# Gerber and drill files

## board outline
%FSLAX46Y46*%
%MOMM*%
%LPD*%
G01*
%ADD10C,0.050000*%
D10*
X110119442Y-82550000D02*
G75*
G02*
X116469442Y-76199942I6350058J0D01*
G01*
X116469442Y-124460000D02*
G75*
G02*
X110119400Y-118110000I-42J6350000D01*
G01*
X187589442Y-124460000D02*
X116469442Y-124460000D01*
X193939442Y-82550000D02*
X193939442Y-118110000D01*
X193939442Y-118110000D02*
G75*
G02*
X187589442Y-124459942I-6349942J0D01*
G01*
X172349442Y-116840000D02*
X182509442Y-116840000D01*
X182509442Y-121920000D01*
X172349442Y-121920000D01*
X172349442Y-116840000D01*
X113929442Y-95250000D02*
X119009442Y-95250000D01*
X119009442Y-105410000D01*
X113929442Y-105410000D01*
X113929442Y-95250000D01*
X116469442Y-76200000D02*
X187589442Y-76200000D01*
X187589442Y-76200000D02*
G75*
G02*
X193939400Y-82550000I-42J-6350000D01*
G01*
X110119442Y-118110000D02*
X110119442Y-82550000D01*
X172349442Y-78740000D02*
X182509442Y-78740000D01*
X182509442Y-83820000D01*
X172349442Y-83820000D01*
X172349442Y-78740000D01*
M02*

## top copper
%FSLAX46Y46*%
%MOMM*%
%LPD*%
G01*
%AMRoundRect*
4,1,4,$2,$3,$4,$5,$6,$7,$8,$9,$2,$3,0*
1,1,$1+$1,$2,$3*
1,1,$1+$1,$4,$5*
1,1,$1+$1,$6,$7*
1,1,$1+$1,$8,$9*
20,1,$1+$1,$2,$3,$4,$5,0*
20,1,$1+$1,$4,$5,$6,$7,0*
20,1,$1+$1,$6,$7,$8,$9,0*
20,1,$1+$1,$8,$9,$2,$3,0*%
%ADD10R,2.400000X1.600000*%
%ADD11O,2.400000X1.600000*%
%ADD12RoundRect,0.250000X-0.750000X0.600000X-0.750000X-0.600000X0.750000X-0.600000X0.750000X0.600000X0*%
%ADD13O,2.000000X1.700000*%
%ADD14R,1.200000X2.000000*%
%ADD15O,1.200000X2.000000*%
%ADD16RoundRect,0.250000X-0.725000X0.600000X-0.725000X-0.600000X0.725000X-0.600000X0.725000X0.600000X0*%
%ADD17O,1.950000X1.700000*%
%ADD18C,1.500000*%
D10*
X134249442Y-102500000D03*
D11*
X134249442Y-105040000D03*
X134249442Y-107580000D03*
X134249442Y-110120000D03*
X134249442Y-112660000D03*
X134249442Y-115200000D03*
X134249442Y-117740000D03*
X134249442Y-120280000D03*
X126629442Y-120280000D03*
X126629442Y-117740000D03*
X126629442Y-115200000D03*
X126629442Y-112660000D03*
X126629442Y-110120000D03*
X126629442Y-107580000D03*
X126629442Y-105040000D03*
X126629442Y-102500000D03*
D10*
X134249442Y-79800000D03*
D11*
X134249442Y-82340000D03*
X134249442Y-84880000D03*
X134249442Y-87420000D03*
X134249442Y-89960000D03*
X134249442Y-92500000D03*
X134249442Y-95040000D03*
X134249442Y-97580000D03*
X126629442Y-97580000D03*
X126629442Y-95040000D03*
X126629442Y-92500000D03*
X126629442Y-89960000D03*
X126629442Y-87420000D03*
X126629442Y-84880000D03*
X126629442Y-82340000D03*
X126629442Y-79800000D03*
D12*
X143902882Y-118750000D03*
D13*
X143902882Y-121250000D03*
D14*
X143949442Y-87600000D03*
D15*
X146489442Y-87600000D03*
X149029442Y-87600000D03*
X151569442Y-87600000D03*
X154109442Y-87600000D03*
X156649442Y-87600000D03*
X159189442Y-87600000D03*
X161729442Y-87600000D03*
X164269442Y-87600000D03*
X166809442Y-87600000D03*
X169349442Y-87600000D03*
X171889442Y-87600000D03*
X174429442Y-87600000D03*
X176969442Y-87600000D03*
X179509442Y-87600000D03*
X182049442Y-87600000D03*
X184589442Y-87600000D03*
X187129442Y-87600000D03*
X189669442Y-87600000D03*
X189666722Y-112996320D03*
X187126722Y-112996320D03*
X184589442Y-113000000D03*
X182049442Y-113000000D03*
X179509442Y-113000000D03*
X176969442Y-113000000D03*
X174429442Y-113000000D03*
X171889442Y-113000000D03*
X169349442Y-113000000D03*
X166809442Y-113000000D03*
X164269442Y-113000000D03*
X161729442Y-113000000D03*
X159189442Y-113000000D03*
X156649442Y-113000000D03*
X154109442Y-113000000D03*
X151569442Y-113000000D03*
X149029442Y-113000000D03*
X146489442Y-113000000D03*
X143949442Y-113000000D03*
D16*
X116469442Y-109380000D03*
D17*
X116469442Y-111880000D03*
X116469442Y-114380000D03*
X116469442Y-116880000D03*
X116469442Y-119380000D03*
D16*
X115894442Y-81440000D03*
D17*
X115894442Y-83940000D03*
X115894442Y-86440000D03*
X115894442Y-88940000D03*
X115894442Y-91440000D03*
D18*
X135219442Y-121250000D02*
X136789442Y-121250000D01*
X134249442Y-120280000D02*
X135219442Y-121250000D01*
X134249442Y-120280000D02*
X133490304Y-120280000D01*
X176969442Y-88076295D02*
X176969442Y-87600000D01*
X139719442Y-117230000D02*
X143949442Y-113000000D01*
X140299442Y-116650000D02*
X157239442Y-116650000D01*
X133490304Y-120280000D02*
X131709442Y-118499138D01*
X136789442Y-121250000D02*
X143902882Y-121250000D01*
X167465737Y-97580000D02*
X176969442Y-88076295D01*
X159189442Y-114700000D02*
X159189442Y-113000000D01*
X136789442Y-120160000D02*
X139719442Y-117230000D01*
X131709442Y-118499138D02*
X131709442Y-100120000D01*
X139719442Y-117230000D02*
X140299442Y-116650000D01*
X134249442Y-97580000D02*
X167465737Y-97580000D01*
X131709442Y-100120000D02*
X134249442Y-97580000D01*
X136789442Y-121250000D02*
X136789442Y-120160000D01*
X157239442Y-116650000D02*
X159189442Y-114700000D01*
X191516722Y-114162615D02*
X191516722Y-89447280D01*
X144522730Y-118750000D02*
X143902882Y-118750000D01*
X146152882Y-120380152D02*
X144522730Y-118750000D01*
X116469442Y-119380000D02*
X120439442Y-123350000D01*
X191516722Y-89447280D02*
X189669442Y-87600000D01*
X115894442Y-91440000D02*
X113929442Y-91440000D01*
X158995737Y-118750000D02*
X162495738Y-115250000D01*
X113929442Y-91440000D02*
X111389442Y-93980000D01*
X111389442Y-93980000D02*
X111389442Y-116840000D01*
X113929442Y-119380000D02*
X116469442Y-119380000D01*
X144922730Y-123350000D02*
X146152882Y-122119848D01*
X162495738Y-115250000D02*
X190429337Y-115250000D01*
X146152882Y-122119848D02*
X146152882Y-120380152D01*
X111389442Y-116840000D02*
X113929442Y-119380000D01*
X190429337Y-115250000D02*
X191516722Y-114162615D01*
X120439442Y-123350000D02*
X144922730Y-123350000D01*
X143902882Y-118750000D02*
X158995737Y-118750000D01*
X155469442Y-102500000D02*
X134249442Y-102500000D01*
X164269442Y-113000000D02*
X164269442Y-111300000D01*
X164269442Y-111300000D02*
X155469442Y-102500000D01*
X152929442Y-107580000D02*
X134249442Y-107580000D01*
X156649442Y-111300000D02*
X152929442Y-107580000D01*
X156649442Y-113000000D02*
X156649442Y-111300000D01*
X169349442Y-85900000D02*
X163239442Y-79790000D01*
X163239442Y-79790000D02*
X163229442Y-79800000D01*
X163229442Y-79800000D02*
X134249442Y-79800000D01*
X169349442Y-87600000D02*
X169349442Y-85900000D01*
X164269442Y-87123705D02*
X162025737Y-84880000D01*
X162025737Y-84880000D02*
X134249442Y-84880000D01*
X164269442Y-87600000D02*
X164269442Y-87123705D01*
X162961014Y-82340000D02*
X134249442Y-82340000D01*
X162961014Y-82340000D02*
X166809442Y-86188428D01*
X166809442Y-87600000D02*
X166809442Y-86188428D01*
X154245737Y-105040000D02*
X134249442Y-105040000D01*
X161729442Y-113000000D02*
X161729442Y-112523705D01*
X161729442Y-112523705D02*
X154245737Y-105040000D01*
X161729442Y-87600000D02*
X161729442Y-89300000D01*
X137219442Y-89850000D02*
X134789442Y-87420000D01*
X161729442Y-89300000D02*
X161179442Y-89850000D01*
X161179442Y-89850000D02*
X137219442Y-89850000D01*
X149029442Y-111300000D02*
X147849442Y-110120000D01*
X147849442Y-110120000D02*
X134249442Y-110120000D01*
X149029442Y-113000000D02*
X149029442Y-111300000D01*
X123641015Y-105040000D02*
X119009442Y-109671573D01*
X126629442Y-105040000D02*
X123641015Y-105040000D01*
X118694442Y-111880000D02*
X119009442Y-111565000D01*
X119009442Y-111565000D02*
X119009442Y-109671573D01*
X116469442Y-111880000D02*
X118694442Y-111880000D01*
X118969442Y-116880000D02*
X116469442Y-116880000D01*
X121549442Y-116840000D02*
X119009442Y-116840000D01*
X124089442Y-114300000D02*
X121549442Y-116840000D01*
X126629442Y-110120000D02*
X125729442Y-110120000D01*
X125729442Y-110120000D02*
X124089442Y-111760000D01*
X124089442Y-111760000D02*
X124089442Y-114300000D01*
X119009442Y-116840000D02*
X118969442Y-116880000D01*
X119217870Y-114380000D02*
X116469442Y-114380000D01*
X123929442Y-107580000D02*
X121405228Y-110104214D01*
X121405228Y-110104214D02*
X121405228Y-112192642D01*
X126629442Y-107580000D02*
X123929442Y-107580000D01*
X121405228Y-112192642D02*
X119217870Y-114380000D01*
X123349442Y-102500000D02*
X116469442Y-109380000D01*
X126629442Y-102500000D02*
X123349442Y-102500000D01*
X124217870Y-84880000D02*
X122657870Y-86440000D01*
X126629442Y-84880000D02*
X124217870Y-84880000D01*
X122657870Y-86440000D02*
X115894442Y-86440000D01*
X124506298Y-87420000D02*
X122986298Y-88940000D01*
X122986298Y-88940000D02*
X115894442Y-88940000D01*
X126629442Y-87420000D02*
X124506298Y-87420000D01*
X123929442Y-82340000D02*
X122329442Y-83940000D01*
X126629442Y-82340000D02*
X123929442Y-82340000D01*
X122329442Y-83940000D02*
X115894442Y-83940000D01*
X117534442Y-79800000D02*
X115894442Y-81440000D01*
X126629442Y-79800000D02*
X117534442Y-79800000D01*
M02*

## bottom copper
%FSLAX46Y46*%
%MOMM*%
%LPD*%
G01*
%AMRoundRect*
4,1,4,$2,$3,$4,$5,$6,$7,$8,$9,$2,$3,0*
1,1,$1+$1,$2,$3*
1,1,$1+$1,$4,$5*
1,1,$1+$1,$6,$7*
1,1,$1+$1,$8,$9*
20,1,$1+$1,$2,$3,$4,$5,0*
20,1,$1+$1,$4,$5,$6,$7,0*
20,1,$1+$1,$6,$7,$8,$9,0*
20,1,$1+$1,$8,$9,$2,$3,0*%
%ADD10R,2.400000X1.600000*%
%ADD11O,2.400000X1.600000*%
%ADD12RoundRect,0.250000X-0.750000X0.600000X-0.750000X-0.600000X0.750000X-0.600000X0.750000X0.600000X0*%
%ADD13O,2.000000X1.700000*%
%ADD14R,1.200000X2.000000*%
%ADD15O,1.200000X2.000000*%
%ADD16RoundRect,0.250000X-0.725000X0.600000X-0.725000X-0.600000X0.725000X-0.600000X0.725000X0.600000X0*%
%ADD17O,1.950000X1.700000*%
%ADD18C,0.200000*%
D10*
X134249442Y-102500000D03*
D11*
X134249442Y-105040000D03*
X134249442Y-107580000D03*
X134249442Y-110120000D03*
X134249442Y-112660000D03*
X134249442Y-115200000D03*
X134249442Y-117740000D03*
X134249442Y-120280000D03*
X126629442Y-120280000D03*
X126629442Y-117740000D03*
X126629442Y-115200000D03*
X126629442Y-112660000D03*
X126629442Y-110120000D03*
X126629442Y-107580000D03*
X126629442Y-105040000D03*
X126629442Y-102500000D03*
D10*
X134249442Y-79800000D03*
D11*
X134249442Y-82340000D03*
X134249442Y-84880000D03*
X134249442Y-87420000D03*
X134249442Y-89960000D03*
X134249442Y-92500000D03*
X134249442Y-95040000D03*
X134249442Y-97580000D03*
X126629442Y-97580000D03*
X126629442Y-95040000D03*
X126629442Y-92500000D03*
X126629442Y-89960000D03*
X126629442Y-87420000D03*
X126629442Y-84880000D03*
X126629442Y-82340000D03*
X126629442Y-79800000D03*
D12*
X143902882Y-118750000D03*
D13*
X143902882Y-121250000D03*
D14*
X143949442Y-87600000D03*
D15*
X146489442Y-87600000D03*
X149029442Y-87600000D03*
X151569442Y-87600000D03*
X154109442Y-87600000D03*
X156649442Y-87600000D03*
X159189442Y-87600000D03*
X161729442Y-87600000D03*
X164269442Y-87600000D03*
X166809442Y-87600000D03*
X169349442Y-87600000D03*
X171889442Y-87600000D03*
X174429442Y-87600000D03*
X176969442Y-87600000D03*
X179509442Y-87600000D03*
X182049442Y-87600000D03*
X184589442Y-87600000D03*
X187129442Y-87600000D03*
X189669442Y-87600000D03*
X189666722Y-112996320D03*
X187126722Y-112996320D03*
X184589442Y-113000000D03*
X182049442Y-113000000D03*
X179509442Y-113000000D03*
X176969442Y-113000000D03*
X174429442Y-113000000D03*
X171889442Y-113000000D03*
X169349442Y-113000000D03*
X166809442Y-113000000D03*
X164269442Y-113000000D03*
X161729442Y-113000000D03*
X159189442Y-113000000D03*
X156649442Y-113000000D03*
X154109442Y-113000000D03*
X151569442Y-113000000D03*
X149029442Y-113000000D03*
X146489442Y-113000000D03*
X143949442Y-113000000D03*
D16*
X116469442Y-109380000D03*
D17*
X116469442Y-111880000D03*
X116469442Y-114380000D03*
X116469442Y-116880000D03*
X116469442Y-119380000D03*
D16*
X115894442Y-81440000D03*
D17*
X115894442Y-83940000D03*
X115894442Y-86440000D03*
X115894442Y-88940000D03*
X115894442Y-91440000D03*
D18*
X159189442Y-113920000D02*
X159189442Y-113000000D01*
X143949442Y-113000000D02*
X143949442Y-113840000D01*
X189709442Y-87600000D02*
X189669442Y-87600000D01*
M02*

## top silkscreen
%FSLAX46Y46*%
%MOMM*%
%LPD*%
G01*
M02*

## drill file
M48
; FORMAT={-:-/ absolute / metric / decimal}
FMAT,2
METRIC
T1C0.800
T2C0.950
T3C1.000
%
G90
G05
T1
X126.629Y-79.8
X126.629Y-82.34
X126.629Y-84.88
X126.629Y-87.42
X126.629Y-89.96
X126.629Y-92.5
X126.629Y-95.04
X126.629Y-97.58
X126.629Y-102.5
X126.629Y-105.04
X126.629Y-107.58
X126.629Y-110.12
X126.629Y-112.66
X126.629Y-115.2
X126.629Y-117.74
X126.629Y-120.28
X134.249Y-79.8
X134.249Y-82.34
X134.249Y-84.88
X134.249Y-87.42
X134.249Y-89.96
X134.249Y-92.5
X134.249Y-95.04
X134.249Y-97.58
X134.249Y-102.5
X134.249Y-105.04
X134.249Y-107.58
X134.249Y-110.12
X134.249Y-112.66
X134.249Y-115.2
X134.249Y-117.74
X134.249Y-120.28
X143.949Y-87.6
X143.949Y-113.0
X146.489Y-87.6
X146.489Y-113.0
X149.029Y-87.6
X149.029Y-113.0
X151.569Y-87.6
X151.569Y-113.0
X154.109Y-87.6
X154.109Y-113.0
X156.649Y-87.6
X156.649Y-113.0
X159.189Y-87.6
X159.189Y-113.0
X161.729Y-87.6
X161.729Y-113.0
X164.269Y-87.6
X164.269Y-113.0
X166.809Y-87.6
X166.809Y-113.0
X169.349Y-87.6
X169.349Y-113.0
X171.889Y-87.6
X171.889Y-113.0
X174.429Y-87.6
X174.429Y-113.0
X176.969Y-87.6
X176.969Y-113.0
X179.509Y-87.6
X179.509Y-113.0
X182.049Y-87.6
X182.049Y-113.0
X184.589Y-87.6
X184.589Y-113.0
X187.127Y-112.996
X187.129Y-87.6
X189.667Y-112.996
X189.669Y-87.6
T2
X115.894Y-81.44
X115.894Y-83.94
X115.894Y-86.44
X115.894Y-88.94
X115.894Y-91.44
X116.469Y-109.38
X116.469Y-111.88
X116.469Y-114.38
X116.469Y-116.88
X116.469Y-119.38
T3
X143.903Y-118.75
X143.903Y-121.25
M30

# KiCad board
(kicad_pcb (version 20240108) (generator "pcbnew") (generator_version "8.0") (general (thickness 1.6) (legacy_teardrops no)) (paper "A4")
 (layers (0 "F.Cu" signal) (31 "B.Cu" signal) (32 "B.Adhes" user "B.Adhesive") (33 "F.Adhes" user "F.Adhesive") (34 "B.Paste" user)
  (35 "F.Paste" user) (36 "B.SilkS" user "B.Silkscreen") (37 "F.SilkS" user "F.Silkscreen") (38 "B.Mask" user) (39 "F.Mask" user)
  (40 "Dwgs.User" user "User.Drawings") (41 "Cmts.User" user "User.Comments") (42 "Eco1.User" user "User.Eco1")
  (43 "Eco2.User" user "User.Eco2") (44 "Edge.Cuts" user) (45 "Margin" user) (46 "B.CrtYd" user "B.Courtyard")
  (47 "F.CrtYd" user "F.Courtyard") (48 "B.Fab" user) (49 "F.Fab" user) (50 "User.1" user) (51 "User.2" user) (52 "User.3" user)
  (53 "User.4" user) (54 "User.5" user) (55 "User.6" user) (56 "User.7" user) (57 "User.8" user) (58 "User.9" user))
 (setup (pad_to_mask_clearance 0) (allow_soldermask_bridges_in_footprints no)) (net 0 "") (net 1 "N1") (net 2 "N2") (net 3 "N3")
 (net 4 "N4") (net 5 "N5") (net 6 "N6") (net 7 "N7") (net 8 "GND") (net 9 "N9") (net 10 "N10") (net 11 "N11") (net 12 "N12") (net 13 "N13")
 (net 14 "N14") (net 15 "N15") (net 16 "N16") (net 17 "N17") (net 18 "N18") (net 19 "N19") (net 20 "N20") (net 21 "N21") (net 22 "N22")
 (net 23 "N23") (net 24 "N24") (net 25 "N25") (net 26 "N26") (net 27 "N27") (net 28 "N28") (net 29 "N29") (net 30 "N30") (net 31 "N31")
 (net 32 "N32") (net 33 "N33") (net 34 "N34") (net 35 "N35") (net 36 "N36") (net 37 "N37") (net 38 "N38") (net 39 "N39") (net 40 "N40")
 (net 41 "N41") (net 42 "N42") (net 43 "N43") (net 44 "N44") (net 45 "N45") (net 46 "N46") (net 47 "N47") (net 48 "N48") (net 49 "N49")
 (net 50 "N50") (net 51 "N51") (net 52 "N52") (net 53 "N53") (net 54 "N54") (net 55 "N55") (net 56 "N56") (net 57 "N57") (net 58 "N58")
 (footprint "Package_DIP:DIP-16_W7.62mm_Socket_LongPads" (layer "B.Cu") (at 134.249442 102.5 180)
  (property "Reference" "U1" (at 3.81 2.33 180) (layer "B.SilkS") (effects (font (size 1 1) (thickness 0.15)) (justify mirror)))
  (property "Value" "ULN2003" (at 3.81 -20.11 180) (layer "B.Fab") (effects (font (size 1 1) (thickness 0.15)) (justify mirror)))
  (pad "1" thru_hole rect (at 0 0 180) (size 2.4 1.6) (drill 0.8) (layers "*.Cu" "*.Mask") (remove_unused_layers no) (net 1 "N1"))
  (pad "2" thru_hole oval (at 0 -2.54 180) (size 2.4 1.6) (drill 0.8) (layers "*.Cu" "*.Mask") (remove_unused_layers no) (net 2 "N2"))
  (pad "3" thru_hole oval (at 0 -5.08 180) (size 2.4 1.6) (drill 0.8) (layers "*.Cu" "*.Mask") (remove_unused_layers no) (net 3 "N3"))
  (pad "4" thru_hole oval (at 0 -7.62 180) (size 2.4 1.6) (drill 0.8) (layers "*.Cu" "*.Mask") (remove_unused_layers no) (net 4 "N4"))
  (pad "5" thru_hole oval (at 0 -10.16 180) (size 2.4 1.6) (drill 0.8) (layers "*.Cu" "*.Mask") (remove_unused_layers no) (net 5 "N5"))
  (pad "6" thru_hole oval (at 0 -12.7 180) (size 2.4 1.6) (drill 0.8) (layers "*.Cu" "*.Mask") (remove_unused_layers no) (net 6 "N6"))
  (pad "7" thru_hole oval (at 0 -15.24 180) (size 2.4 1.6) (drill 0.8) (layers "*.Cu" "*.Mask") (remove_unused_layers no) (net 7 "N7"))
  (pad "8" thru_hole oval (at 0 -17.78 180) (size 2.4 1.6) (drill 0.8) (layers "*.Cu" "*.Mask") (remove_unused_layers no) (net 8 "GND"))
  (pad "9" thru_hole oval (at 7.62 -17.78 180) (size 2.4 1.6) (drill 0.8) (layers "*.Cu" "*.Mask") (remove_unused_layers no) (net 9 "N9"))
  (pad "10" thru_hole oval (at 7.62 -15.24 180) (size 2.4 1.6) (drill 0.8) (layers "*.Cu" "*.Mask") (remove_unused_layers no) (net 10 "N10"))
  (pad "11" thru_hole oval (at 7.62 -12.7 180) (size 2.4 1.6) (drill 0.8) (layers "*.Cu" "*.Mask") (remove_unused_layers no) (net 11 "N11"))
  (pad "12" thru_hole oval (at 7.62 -10.16 180) (size 2.4 1.6) (drill 0.8) (layers "*.Cu" "*.Mask") (remove_unused_layers no) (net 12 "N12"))
  (pad "13" thru_hole oval (at 7.62 -7.62 180) (size 2.4 1.6) (drill 0.8) (layers "*.Cu" "*.Mask") (remove_unused_layers no) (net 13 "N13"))
  (pad "14" thru_hole oval (at 7.62 -5.08 180) (size 2.4 1.6) (drill 0.8) (layers "*.Cu" "*.Mask") (remove_unused_layers no) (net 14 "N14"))
  (pad "15" thru_hole oval (at 7.62 -2.54 180) (size 2.4 1.6) (drill 0.8) (layers "*.Cu" "*.Mask") (remove_unused_layers no) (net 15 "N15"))
  (pad "16" thru_hole oval (at 7.62 0 180) (size 2.4 1.6) (drill 0.8) (layers "*.Cu" "*.Mask") (remove_unused_layers no) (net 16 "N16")))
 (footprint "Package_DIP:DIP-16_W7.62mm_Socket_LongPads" (layer "B.Cu") (at 134.249442 79.8 180)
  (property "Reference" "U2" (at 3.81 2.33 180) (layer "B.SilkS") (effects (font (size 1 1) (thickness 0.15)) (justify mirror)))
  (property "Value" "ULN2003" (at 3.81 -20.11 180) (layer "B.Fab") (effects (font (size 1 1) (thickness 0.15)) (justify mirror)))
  (pad "1" thru_hole rect (at 0 0 180) (size 2.4 1.6) (drill 0.8) (layers "*.Cu" "*.Mask") (remove_unused_layers no) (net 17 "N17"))
  (pad "2" thru_hole oval (at 0 -2.54 180) (size 2.4 1.6) (drill 0.8) (layers "*.Cu" "*.Mask") (remove_unused_layers no) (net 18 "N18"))
  (pad "3" thru_hole oval (at 0 -5.08 180) (size 2.4 1.6) (drill 0.8) (layers "*.Cu" "*.Mask") (remove_unused_layers no) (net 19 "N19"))
  (pad "4" thru_hole oval (at 0 -7.62 180) (size 2.4 1.6) (drill 0.8) (layers "*.Cu" "*.Mask") (remove_unused_layers no) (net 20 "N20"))
  (pad "5" thru_hole oval (at 0 -10.16 180) (size 2.4 1.6) (drill 0.8) (layers "*.Cu" "*.Mask") (remove_unused_layers no) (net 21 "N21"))
  (pad "6" thru_hole oval (at 0 -12.7 180) (size 2.4 1.6) (drill 0.8) (layers "*.Cu" "*.Mask") (remove_unused_layers no) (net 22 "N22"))
  (pad "7" thru_hole oval (at 0 -15.24 180) (size 2.4 1.6) (drill 0.8) (layers "*.Cu" "*.Mask") (remove_unused_layers no) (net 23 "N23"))
  (pad "8" thru_hole oval (at 0 -17.78 180) (size 2.4 1.6) (drill 0.8) (layers "*.Cu" "*.Mask") (remove_unused_layers no) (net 8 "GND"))
  (pad "9" thru_hole oval (at 7.62 -17.78 180) (size 2.4 1.6) (drill 0.8) (layers "*.Cu" "*.Mask") (remove_unused_layers no) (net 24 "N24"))
  (pad "10" thru_hole oval (at 7.62 -15.24 180) (size 2.4 1.6) (drill 0.8) (layers "*.Cu" "*.Mask") (remove_unused_layers no) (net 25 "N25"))
  (pad "11" thru_hole oval (at 7.62 -12.7 180) (size 2.4 1.6) (drill 0.8) (layers "*.Cu" "*.Mask") (remove_unused_layers no) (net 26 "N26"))
  (pad "12" thru_hole oval (at 7.62 -10.16 180) (size 2.4 1.6) (drill 0.8) (layers "*.Cu" "*.Mask") (remove_unused_layers no) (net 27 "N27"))
  (pad "13" thru_hole oval (at 7.62 -7.62 180) (size 2.4 1.6) (drill 0.8) (layers "*.Cu" "*.Mask") (remove_unused_layers no) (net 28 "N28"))
  (pad "14" thru_hole oval (at 7.62 -5.08 180) (size 2.4 1.6) (drill 0.8) (layers "*.Cu" "*.Mask") (remove_unused_layers no) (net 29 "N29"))
  (pad "15" thru_hole oval (at 7.62 -2.54 180) (size 2.4 1.6) (drill 0.8) (layers "*.Cu" "*.Mask") (remove_unused_layers no) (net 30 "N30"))
  (pad "16" thru_hole oval (at 7.62 0 180) (size 2.4 1.6) (drill 0.8) (layers "*.Cu" "*.Mask") (remove_unused_layers no) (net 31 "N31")))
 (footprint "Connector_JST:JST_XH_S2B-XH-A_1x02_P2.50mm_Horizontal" (layer "B.Cu") (at 143.902882 118.75 -90)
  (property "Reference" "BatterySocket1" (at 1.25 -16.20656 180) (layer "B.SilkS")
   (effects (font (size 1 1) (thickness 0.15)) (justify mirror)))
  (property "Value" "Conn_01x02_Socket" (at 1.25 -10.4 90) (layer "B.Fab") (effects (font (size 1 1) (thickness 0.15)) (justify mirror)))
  (pad "1" thru_hole roundrect (at 0 0 270) (size 1.7 2) (drill 1) (layers "*.Cu" "*.Mask") (remove_unused_layers no)
   (roundrect_rratio 0.1470588235) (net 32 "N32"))
  (pad "2" thru_hole oval (at 2.5 0 270) (size 1.7 2) (drill 1) (layers "*.Cu" "*.Mask") (remove_unused_layers no) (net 8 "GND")))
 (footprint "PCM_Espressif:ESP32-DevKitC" (layer "B.Cu") (at 143.949442 87.6 -90)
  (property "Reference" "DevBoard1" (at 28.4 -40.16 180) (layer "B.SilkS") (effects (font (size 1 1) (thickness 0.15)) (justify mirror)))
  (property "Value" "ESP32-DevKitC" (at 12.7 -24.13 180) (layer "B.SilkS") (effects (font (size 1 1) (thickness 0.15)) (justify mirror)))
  (pad "1" thru_hole rect (at 0 0) (size 1.2 2) (drill 0.8) (layers "*.Cu" "*.Mask") (remove_unused_layers no) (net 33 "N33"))
  (pad "2" thru_hole oval (at 0 -2.54) (size 1.2 2) (drill 0.8) (layers "*.Cu" "*.Mask") (remove_unused_layers no) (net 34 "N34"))
  (pad "3" thru_hole oval (at 0 -5.08) (size 1.2 2) (drill 0.8) (layers "*.Cu" "*.Mask") (remove_unused_layers no) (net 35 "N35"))
  (pad "4" thru_hole oval (at 0 -7.62) (size 1.2 2) (drill 0.8) (layers "*.Cu" "*.Mask") (remove_unused_layers no) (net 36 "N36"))
  (pad "5" thru_hole oval (at 0 -10.16) (size 1.2 2) (drill 0.8) (layers "*.Cu" "*.Mask") (remove_unused_layers no) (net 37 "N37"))
  (pad "6" thru_hole oval (at 0 -12.7) (size 1.2 2) (drill 0.8) (layers "*.Cu" "*.Mask") (remove_unused_layers no) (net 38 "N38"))
  (pad "7" thru_hole oval (at 0 -15.24) (size 1.2 2) (drill 0.8) (layers "*.Cu" "*.Mask") (remove_unused_layers no) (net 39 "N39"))
  (pad "8" thru_hole oval (at 0 -17.78) (size 1.2 2) (drill 0.8) (layers "*.Cu" "*.Mask") (remove_unused_layers no) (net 20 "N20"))
  (pad "9" thru_hole oval (at 0 -20.32) (size 1.2 2) (drill 0.8) (layers "*.Cu" "*.Mask") (remove_unused_layers no) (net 19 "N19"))
  (pad "10" thru_hole oval (at 0 -22.86) (size 1.2 2) (drill 0.8) (layers "*.Cu" "*.Mask") (remove_unused_layers no) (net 18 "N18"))
  (pad "11" thru_hole oval (at 0 -25.4) (size 1.2 2) (drill 0.8) (layers "*.Cu" "*.Mask") (remove_unused_layers no) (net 17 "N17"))
  (pad "12" thru_hole oval (at 0 -27.94) (size 1.2 2) (drill 0.8) (layers "*.Cu" "*.Mask") (remove_unused_layers no) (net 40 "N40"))
  (pad "13" thru_hole oval (at 0 -30.48) (size 1.2 2) (drill 0.8) (layers "*.Cu" "*.Mask") (remove_unused_layers no) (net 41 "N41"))
  (pad "14" thru_hole oval (at 0 -33.02) (size 1.2 2) (drill 0.8) (layers "*.Cu" "*.Mask") (remove_unused_layers no) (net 8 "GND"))
  (pad "15" thru_hole oval (at 0 -35.56) (size 1.2 2) (drill 0.8) (layers "*.Cu" "*.Mask") (remove_unused_layers no) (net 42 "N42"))
  (pad "16" thru_hole oval (at 0 -38.1) (size 1.2 2) (drill 0.8) (layers "*.Cu" "*.Mask") (remove_unused_layers no) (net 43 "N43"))
  (pad "17" thru_hole oval (at 0 -40.64) (size 1.2 2) (drill 0.8) (layers "*.Cu" "*.Mask") (remove_unused_layers no) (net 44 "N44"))
  (pad "18" thru_hole oval (at 0 -43.18) (size 1.2 2) (drill 0.8) (layers "*.Cu" "*.Mask") (remove_unused_layers no) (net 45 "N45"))
  (pad "19" thru_hole oval (at 0 -45.72) (size 1.2 2) (drill 0.8) (layers "*.Cu" "*.Mask") (remove_unused_layers no) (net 32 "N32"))
  (pad "20" thru_hole oval (at 25.39632 -45.71728) (size 1.2 2) (drill 0.8) (layers "*.Cu" "*.Mask") (remove_unused_layers no)
   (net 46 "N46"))
  (pad "21" thru_hole oval (at 25.39632 -43.17728) (size 1.2 2) (drill 0.8) (layers "*.Cu" "*.Mask") (remove_unused_layers no)
   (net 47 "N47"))
  (pad "22" thru_hole oval (at 25.4 -40.64) (size 1.2 2) (drill 0.8) (layers "*.Cu" "*.Mask") (remove_unused_layers no) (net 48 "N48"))
  (pad "23" thru_hole oval (at 25.4 -38.1) (size 1.2 2) (drill 0.8) (layers "*.Cu" "*.Mask") (remove_unused_layers no) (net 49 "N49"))
  (pad "24" thru_hole oval (at 25.4 -35.56) (size 1.2 2) (drill 0.8) (layers "*.Cu" "*.Mask") (remove_unused_layers no) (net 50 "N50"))
  (pad "25" thru_hole oval (at 25.4 -33.02) (size 1.2 2) (drill 0.8) (layers "*.Cu" "*.Mask") (remove_unused_layers no) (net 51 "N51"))
  (pad "26" thru_hole oval (at 25.4 -30.48) (size 1.2 2) (drill 0.8) (layers "*.Cu" "*.Mask") (remove_unused_layers no) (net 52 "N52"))
  (pad "27" thru_hole oval (at 25.4 -27.94) (size 1.2 2) (drill 0.8) (layers "*.Cu" "*.Mask") (remove_unused_layers no) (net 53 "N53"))
  (pad "28" thru_hole oval (at 25.4 -25.4) (size 1.2 2) (drill 0.8) (layers "*.Cu" "*.Mask") (remove_unused_layers no) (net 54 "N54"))
  (pad "29" thru_hole oval (at 25.4 -22.86) (size 1.2 2) (drill 0.8) (layers "*.Cu" "*.Mask") (remove_unused_layers no) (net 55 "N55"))
  (pad "30" thru_hole oval (at 25.4 -20.32) (size 1.2 2) (drill 0.8) (layers "*.Cu" "*.Mask") (remove_unused_layers no) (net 1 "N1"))
  (pad "31" thru_hole oval (at 25.4 -17.78) (size 1.2 2) (drill 0.8) (layers "*.Cu" "*.Mask") (remove_unused_layers no) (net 2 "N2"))
  (pad "32" thru_hole oval (at 25.4 -15.24) (size 1.2 2) (drill 0.8) (layers "*.Cu" "*.Mask") (remove_unused_layers no) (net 8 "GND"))
  (pad "33" thru_hole oval (at 25.4 -12.7) (size 1.2 2) (drill 0.8) (layers "*.Cu" "*.Mask") (remove_unused_layers no) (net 3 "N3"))
  (pad "34" thru_hole oval (at 25.4 -10.16) (size 1.2 2) (drill 0.8) (layers "*.Cu" "*.Mask") (remove_unused_layers no) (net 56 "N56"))
  (pad "35" thru_hole oval (at 25.4 -7.62) (size 1.2 2) (drill 0.8) (layers "*.Cu" "*.Mask") (remove_unused_layers no) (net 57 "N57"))
  (pad "36" thru_hole oval (at 25.4 -5.08) (size 1.2 2) (drill 0.8) (layers "*.Cu" "*.Mask") (remove_unused_layers no) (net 4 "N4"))
  (pad "37" thru_hole oval (at 25.4 -2.54) (size 1.2 2) (drill 0.8) (layers "*.Cu" "*.Mask") (remove_unused_layers no) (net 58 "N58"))
  (pad "38" thru_hole oval (at 25.4 0) (size 1.2 2) (drill 0.8) (layers "*.Cu" "*.Mask") (remove_unused_layers no) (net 8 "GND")))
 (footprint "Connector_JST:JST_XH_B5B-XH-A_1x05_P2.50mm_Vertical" (layer "B.Cu") (at 116.469442 109.38 -90)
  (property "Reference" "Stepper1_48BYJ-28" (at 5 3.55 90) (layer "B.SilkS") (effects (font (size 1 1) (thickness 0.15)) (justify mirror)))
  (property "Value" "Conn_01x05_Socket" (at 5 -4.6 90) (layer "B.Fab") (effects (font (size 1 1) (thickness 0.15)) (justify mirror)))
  (pad "1" thru_hole roundrect (at 0 0 270) (size 1.7 1.95) (drill 0.95) (layers "*.Cu" "*.Mask") (remove_unused_layers no)
   (roundrect_rratio 0.1470588235) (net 16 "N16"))
  (pad "2" thru_hole oval (at 2.5 0 270) (size 1.7 1.95) (drill 0.95) (layers "*.Cu" "*.Mask") (remove_unused_layers no) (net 15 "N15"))
  (pad "3" thru_hole oval (at 5 0 270) (size 1.7 1.95) (drill 0.95) (layers "*.Cu" "*.Mask") (remove_unused_layers no) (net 14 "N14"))
  (pad "4" thru_hole oval (at 7.5 0 270) (size 1.7 1.95) (drill 0.95) (layers "*.Cu" "*.Mask") (remove_unused_layers no) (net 13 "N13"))
  (pad "5" thru_hole oval (at 10 0 270) (size 1.7 1.95) (drill 0.95) (layers "*.Cu" "*.Mask") (remove_unused_layers no) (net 32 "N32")))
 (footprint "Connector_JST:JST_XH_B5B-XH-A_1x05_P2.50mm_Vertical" (layer "B.Cu") (at 115.894442 81.44 -90)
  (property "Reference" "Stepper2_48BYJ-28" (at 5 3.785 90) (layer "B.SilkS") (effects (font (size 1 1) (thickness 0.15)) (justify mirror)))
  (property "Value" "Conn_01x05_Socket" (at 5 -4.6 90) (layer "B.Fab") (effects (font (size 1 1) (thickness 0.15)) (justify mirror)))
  (pad "1" thru_hole roundrect (at 0 0 270) (size 1.7 1.95) (drill 0.95) (layers "*.Cu" "*.Mask") (remove_unused_layers no)
   (roundrect_rratio 0.1470588235) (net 31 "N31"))
  (pad "2" thru_hole oval (at 2.5 0 270) (size 1.7 1.95) (drill 0.95) (layers "*.Cu" "*.Mask") (remove_unused_layers no) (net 30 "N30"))
  (pad "3" thru_hole oval (at 5 0 270) (size 1.7 1.95) (drill 0.95) (layers "*.Cu" "*.Mask") (remove_unused_layers no) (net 29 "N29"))
  (pad "4" thru_hole oval (at 7.5 0 270) (size 1.7 1.95) (drill 0.95) (layers "*.Cu" "*.Mask") (remove_unused_layers no) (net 28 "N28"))
  (pad "5" thru_hole oval (at 10 0 270) (size 1.7 1.95) (drill 0.95) (layers "*.Cu" "*.Mask") (remove_unused_layers no) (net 32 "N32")))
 (gr_arc (start 110.119442 82.55) (mid 111.979315 78.059877) (end 116.469442 76.2) (stroke (width 0.05) (type default)) (layer "Edge.Cuts"))
 (gr_arc (start 116.469442 124.46) (mid 111.979305 122.600133) (end 110.119442 118.11) (stroke (width 0.05) (type default))
  (layer "Edge.Cuts"))
 (gr_line (start 187.589442 124.46) (end 116.469442 124.46) (stroke (width 0.05) (type default)) (layer "Edge.Cuts"))
 (gr_line (start 193.939442 82.55) (end 193.939442 118.11) (stroke (width 0.05) (type default)) (layer "Edge.Cuts"))
 (gr_arc (start 193.939442 118.11) (mid 192.079571 122.600133) (end 187.589442 124.46) (stroke (width 0.05) (type default))
  (layer "Edge.Cuts"))
 (gr_rect (start 172.349442 116.84) (end 182.509442 121.92) (stroke (width 0.05) (type default)) (fill none) (layer "Edge.Cuts"))
 (gr_rect (start 113.929442 95.25) (end 119.009442 105.41) (stroke (width 0.05) (type default)) (fill none) (layer "Edge.Cuts"))
 (gr_line (start 116.469442 76.2) (end 187.589442 76.2) (stroke (width 0.05) (type default)) (layer "Edge.Cuts"))
 (gr_arc (start 187.589442 76.2) (mid 192.079561 78.059877) (end 193.939442 82.55) (stroke (width 0.05) (type default)) (layer "Edge.Cuts"))
 (gr_line (start 110.119442 118.11) (end 110.119442 82.55) (stroke (width 0.05) (type default)) (layer "Edge.Cuts"))
 (gr_rect (start 172.349442 78.74) (end 182.509442 83.82) (stroke (width 0.05) (type default)) (fill none) (layer "Edge.Cuts"))
 (segment (start 135.219442 121.25) (end 136.789442 121.25) (width 1.5) (layer "F.Cu") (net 8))
 (segment (start 134.249442 120.28) (end 135.219442 121.25) (width 1.5) (layer "F.Cu") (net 8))
 (segment (start 134.249442 120.28) (end 133.490304 120.28) (width 1.5) (layer "F.Cu") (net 8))
 (segment (start 176.969442 88.076295) (end 176.969442 87.6) (width 1.5) (layer "F.Cu") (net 8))
 (segment (start 139.719442 117.23) (end 143.949442 113) (width 1.5) (layer "F.Cu") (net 8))
 (segment (start 140.299442 116.65) (end 157.239442 116.65) (width 1.5) (layer "F.Cu") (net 8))
 (segment (start 133.490304 120.28) (end 131.709442 118.499138) (width 1.5) (layer "F.Cu") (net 8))
 (segment (start 136.789442 121.25) (end 143.902882 121.25) (width 1.5) (layer "F.Cu") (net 8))
 (segment (start 167.465737 97.58) (end 176.969442 88.076295) (width 1.5) (layer "F.Cu") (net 8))
 (segment (start 159.189442 114.7) (end 159.189442 113) (width 1.5) (layer "F.Cu") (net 8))
 (segment (start 136.789442 120.16) (end 139.719442 117.23) (width 1.5) (layer "F.Cu") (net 8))
 (segment (start 131.709442 118.499138) (end 131.709442 100.12) (width 1.5) (layer "F.Cu") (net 8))
 (segment (start 139.719442 117.23) (end 140.299442 116.65) (width 1.5) (layer "F.Cu") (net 8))
 (segment (start 134.249442 97.58) (end 167.465737 97.58) (width 1.5) (layer "F.Cu") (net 8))
 (segment (start 131.709442 100.12) (end 134.249442 97.58) (width 1.5) (layer "F.Cu") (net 8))
 (segment (start 136.789442 121.25) (end 136.789442 120.16) (width 1.5) (layer "F.Cu") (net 8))
 (segment (start 157.239442 116.65) (end 159.189442 114.7) (width 1.5) (layer "F.Cu") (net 8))
 (segment (start 159.189442 113.92) (end 159.189442 113) (width 0.2) (layer "B.Cu") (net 8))
 (segment (start 143.949442 113) (end 143.949442 113.84) (width 0.2) (layer "B.Cu") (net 8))
 (segment (start 191.516722 114.162615) (end 191.516722 89.44728) (width 1.5) (layer "F.Cu") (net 32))
 (segment (start 144.52273 118.75) (end 143.902882 118.75) (width 1.5) (layer "F.Cu") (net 32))
 (segment (start 146.152882 120.380152) (end 144.52273 118.75) (width 1.5) (layer "F.Cu") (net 32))
 (segment (start 116.469442 119.38) (end 120.439442 123.35) (width 1.5) (layer "F.Cu") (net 32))
 (segment (start 191.516722 89.44728) (end 189.669442 87.6) (width 1.5) (layer "F.Cu") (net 32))
 (segment (start 115.894442 91.44) (end 113.929442 91.44) (width 1.5) (layer "F.Cu") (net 32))
 (segment (start 158.995737 118.75) (end 162.495738 115.25) (width 1.5) (layer "F.Cu") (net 32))
 (segment (start 113.929442 91.44) (end 111.389442 93.98) (width 1.5) (layer "F.Cu") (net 32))
 (segment (start 111.389442 93.98) (end 111.389442 116.84) (width 1.5) (layer "F.Cu") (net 32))
 (segment (start 113.929442 119.38) (end 116.469442 119.38) (width 1.5) (layer "F.Cu") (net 32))
 (segment (start 144.92273 123.35) (end 146.152882 122.119848) (width 1.5) (layer "F.Cu") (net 32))
 (segment (start 162.495738 115.25) (end 190.429337 115.25) (width 1.5) (layer "F.Cu") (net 32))
 (segment (start 146.152882 122.119848) (end 146.152882 120.380152) (width 1.5) (layer "F.Cu") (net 32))
 (segment (start 111.389442 116.84) (end 113.929442 119.38) (width 1.5) (layer "F.Cu") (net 32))
 (segment (start 190.429337 115.25) (end 191.516722 114.162615) (width 1.5) (layer "F.Cu") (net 32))
 (segment (start 120.439442 123.35) (end 144.92273 123.35) (width 1.5) (layer "F.Cu") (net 32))
 (segment (start 143.902882 118.75) (end 158.995737 118.75) (width 1.5) (layer "F.Cu") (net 32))
 (segment (start 189.709442 87.6) (end 189.669442 87.6) (width 0.2) (layer "B.Cu") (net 32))
 (segment (start 155.469442 102.5) (end 134.249442 102.5) (width 1.5) (layer "F.Cu") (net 1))
 (segment (start 164.269442 113) (end 164.269442 111.3) (width 1.5) (layer "F.Cu") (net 1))
 (segment (start 164.269442 111.3) (end 155.469442 102.5) (width 1.5) (layer "F.Cu") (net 1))
 (segment (start 152.929442 107.58) (end 134.249442 107.58) (width 1.5) (layer "F.Cu") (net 3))
 (segment (start 156.649442 111.3) (end 152.929442 107.58) (width 1.5) (layer "F.Cu") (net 3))
 (segment (start 156.649442 113) (end 156.649442 111.3) (width 1.5) (layer "F.Cu") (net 3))
 (segment (start 169.349442 85.9) (end 163.239442 79.79) (width 1.5) (layer "F.Cu") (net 17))
 (segment (start 163.239442 79.79) (end 163.229442 79.8) (width 1.5) (layer "F.Cu") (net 17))
 (segment (start 163.229442 79.8) (end 134.249442 79.8) (width 1.5) (layer "F.Cu") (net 17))
 (segment (start 169.349442 87.6) (end 169.349442 85.9) (width 1.5) (layer "F.Cu") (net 17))
 (segment (start 164.269442 87.123705) (end 162.025737 84.88) (width 1.5) (layer "F.Cu") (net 19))
 (segment (start 162.025737 84.88) (end 134.249442 84.88) (width 1.5) (layer "F.Cu") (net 19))
 (segment (start 164.269442 87.6) (end 164.269442 87.123705) (width 1.5) (layer "F.Cu") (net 19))
 (segment (start 162.961014 82.34) (end 134.249442 82.34) (width 1.5) (layer "F.Cu") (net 18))
 (segment (start 162.961014 82.34) (end 166.809442 86.188428) (width 1.5) (layer "F.Cu") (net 18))
 (segment (start 166.809442 87.6) (end 166.809442 86.188428) (width 1.5) (layer "F.Cu") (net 18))
 (segment (start 154.245737 105.04) (end 134.249442 105.04) (width 1.5) (layer "F.Cu") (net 2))
 (segment (start 161.729442 113) (end 161.729442 112.523705) (width 1.5) (layer "F.Cu") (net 2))
 (segment (start 161.729442 112.523705) (end 154.245737 105.04) (width 1.5) (layer "F.Cu") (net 2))
 (segment (start 161.729442 87.6) (end 161.729442 89.3) (width 1.5) (layer "F.Cu") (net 20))
 (segment (start 137.219442 89.85) (end 134.789442 87.42) (width 1.5) (layer "F.Cu") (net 20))
 (segment (start 161.729442 89.3) (end 161.179442 89.85) (width 1.5) (layer "F.Cu") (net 20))
 (segment (start 161.179442 89.85) (end 137.219442 89.85) (width 1.5) (layer "F.Cu") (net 20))
 (segment (start 149.029442 111.3) (end 147.849442 110.12) (width 1.5) (layer "F.Cu") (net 4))
 (segment (start 147.849442 110.12) (end 134.249442 110.12) (width 1.5) (layer "F.Cu") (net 4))
 (segment (start 149.029442 113) (end 149.029442 111.3) (width 1.5) (layer "F.Cu") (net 4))
 (segment (start 123.641015 105.04) (end 119.009442 109.671573) (width 1.5) (layer "F.Cu") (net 15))
 (segment (start 126.629442 105.04) (end 123.641015 105.04) (width 1.5) (layer "F.Cu") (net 15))
 (segment (start 118.694442 111.88) (end 119.009442 111.565) (width 1.5) (layer "F.Cu") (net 15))
 (segment (start 119.009442 111.565) (end 119.009442 109.671573) (width 1.5) (layer "F.Cu") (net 15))
 (segment (start 116.469442 111.88) (end 118.694442 111.88) (width 1.5) (layer "F.Cu") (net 15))
 (segment (start 118.969442 116.88) (end 116.469442 116.88) (width 1.5) (layer "F.Cu") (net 13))
 (segment (start 121.549442 116.84) (end 119.009442 116.84) (width 1.5) (layer "F.Cu") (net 13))
 (segment (start 124.089442 114.3) (end 121.549442 116.84) (width 1.5) (layer "F.Cu") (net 13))
 (segment (start 126.629442 110.12) (end 125.729442 110.12) (width 1.5) (layer "F.Cu") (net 13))
 (segment (start 125.729442 110.12) (end 124.089442 111.76) (width 1.5) (layer "F.Cu") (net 13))
 (segment (start 124.089442 111.76) (end 124.089442 114.3) (width 1.5) (layer "F.Cu") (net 13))
 (segment (start 119.009442 116.84) (end 118.969442 116.88) (width 1.5) (layer "F.Cu") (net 13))
 (segment (start 119.21787 114.38) (end 116.469442 114.38) (width 1.5) (layer "F.Cu") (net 14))
 (segment (start 123.929442 107.58) (end 121.405228 110.104214) (width 1.5) (layer "F.Cu") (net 14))
 (segment (start 121.405228 110.104214) (end 121.405228 112.192642) (width 1.5) (layer "F.Cu") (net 14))
 (segment (start 126.629442 107.58) (end 123.929442 107.58) (width 1.5) (layer "F.Cu") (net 14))
 (segment (start 121.405228 112.192642) (end 119.21787 114.38) (width 1.5) (layer "F.Cu") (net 14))
 (segment (start 123.349442 102.5) (end 116.469442 109.38) (width 1.5) (layer "F.Cu") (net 16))
 (segment (start 126.629442 102.5) (end 123.349442 102.5) (width 1.5) (layer "F.Cu") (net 16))
 (segment (start 124.21787 84.88) (end 122.65787 86.44) (width 1.5) (layer "F.Cu") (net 29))
 (segment (start 126.629442 84.88) (end 124.21787 84.88) (width 1.5) (layer "F.Cu") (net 29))
 (segment (start 122.65787 86.44) (end 115.894442 86.44) (width 1.5) (layer "F.Cu") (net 29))
 (segment (start 124.506298 87.42) (end 122.986298 88.94) (width 1.5) (layer "F.Cu") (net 28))
 (segment (start 122.986298 88.94) (end 115.894442 88.94) (width 1.5) (layer "F.Cu") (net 28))
 (segment (start 126.629442 87.42) (end 124.506298 87.42) (width 1.5) (layer "F.Cu") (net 28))
 (segment (start 123.929442 82.34) (end 122.329442 83.94) (width 1.5) (layer "F.Cu") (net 30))
 (segment (start 126.629442 82.34) (end 123.929442 82.34) (width 1.5) (layer "F.Cu") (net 30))
 (segment (start 122.329442 83.94) (end 115.894442 83.94) (width 1.5) (layer "F.Cu") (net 30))
 (segment (start 117.534442 79.8) (end 115.894442 81.44) (width 1.5) (layer "F.Cu") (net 31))
 (segment (start 126.629442 79.8) (end 117.534442 79.8) (width 1.5) (layer "F.Cu") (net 31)))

